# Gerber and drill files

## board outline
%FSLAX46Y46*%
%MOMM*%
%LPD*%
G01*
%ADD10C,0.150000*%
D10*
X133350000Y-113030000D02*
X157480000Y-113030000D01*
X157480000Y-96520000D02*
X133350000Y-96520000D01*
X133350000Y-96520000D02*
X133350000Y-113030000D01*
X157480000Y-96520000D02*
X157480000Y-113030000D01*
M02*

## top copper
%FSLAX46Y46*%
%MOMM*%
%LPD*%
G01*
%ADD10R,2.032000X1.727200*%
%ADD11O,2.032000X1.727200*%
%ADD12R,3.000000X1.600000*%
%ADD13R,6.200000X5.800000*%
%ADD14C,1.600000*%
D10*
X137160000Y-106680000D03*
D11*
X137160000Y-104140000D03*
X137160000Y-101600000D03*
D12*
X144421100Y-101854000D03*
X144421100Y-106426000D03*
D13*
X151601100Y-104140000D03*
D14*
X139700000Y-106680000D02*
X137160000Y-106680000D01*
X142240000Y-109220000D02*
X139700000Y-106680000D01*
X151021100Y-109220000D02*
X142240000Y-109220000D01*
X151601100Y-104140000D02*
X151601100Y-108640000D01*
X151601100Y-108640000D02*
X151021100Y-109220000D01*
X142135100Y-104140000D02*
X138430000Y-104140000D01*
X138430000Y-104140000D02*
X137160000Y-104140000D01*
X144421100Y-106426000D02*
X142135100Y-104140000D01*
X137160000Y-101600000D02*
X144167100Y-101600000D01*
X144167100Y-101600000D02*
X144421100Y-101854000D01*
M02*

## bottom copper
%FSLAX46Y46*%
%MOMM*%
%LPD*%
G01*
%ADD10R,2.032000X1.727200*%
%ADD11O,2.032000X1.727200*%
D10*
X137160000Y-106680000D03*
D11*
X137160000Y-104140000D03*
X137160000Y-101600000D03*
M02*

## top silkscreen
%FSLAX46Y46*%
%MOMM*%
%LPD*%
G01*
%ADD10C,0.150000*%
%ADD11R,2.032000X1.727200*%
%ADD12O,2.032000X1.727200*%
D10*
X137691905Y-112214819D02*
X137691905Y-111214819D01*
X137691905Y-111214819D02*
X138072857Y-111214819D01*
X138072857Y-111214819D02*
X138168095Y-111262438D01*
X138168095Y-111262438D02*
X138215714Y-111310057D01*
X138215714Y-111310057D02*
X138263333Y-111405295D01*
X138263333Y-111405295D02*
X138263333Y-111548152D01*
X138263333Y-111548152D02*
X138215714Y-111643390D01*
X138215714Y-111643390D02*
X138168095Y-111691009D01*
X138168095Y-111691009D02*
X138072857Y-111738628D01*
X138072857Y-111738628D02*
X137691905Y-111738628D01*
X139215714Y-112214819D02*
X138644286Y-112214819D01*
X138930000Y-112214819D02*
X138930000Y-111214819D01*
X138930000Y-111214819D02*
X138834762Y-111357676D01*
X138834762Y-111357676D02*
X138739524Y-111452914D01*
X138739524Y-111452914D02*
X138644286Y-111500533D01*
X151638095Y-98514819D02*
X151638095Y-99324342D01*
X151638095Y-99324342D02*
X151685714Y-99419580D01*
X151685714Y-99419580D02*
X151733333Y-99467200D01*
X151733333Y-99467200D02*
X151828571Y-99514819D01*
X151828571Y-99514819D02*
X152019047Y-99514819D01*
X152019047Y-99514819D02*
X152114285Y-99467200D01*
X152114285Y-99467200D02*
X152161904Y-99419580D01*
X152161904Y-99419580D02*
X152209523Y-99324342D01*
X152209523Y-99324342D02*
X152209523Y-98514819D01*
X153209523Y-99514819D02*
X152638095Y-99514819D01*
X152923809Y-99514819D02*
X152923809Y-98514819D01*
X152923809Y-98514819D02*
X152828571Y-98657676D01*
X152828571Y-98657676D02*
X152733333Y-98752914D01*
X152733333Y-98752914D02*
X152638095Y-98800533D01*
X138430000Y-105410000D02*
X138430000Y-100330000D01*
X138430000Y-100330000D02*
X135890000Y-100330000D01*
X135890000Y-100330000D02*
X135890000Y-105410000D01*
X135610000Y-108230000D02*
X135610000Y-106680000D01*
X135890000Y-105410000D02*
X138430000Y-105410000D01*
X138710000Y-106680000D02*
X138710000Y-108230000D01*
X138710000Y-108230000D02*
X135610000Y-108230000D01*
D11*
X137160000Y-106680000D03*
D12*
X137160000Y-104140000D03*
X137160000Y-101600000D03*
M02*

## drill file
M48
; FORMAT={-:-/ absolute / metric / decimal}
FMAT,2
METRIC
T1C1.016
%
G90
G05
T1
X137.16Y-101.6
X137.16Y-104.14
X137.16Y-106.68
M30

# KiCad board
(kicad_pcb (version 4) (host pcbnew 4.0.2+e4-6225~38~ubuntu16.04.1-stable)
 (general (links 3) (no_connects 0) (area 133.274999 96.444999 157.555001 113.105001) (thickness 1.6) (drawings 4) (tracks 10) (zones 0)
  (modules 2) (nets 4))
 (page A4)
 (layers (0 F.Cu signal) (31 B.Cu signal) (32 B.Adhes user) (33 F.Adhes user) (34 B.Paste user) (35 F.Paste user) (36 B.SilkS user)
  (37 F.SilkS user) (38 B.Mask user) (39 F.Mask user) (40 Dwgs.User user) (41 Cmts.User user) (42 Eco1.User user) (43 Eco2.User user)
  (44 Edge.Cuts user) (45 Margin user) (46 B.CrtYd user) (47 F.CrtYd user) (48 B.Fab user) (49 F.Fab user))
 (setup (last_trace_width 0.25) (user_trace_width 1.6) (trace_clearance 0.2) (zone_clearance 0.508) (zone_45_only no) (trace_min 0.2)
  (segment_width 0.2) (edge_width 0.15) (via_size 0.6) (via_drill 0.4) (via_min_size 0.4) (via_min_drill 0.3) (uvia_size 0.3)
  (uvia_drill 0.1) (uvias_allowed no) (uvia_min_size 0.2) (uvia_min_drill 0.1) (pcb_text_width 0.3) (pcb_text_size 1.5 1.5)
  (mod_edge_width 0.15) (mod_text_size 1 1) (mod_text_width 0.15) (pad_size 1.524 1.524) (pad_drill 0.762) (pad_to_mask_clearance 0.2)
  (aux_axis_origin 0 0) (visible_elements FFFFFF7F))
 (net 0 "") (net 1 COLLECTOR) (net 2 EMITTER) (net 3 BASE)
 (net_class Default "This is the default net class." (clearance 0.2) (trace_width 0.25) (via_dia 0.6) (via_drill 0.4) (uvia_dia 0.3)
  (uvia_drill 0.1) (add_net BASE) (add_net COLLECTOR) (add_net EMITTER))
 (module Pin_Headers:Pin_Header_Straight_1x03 (layer F.Cu) (at 137.16 106.68 180)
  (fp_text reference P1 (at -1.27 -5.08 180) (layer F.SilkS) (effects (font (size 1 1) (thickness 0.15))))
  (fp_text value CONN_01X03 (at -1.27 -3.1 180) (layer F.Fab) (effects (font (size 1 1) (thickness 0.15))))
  (fp_line (start -1.27 1.27) (end -1.27 6.35) (layer F.SilkS) (width 0.15))
  (fp_line (start -1.27 6.35) (end 1.27 6.35) (layer F.SilkS) (width 0.15))
  (fp_line (start 1.27 6.35) (end 1.27 1.27) (layer F.SilkS) (width 0.15))
  (fp_line (start 1.55 -1.55) (end 1.55 0) (layer F.SilkS) (width 0.15))
  (fp_line (start 1.27 1.27) (end -1.27 1.27) (layer F.SilkS) (width 0.15))
  (fp_line (start -1.55 0) (end -1.55 -1.55) (layer F.SilkS) (width 0.15))
  (fp_line (start -1.55 -1.55) (end 1.55 -1.55) (layer F.SilkS) (width 0.15))
  (pad 1 thru_hole rect (at 0 0 180) (size 2.032 1.7272) (drill 1.016) (layers *.Cu *.Mask F.SilkS) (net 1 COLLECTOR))
  (pad 2 thru_hole oval (at 0 2.54 180) (size 2.032 1.7272) (drill 1.016) (layers *.Cu *.Mask F.SilkS) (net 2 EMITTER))
  (pad 3 thru_hole oval (at 0 5.08 180) (size 2.032 1.7272) (drill 1.016) (layers *.Cu *.Mask F.SilkS) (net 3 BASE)))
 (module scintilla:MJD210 (layer F.Cu) (at 148.5011 104.14 180)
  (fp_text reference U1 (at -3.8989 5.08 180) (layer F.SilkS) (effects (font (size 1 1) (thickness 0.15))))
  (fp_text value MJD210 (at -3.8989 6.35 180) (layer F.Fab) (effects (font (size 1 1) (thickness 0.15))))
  (pad 1 smd rect (at 4.08 2.286 180) (size 3 1.6) (layers F.Cu F.Paste F.Mask) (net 3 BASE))
  (pad 3 smd rect (at 4.08 -2.286 180) (size 3 1.6) (layers F.Cu F.Paste F.Mask) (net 2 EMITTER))
  (pad 4 smd rect (at -3.1 0 180) (size 6.2 5.8) (layers F.Cu F.Paste F.Mask) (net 1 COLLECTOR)))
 (gr_line (start 133.35 113.03) (end 157.48 113.03) (layer Edge.Cuts) (width 0.15))
 (gr_line (start 157.48 96.52) (end 133.35 96.52) (layer Edge.Cuts) (width 0.15))
 (gr_line (start 133.35 96.52) (end 133.35 113.03) (layer Edge.Cuts) (width 0.15))
 (gr_line (start 157.48 96.52) (end 157.48 113.03) (layer Edge.Cuts) (width 0.15))
 (segment (start 139.7 106.68) (end 137.16 106.68) (width 1.6) (layer F.Cu) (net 1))
 (segment (start 142.24 109.22) (end 139.7 106.68) (width 1.6) (layer F.Cu) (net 1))
 (segment (start 151.0211 109.22) (end 142.24 109.22) (width 1.6) (layer F.Cu) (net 1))
 (segment (start 151.6011 104.14) (end 151.6011 108.64) (width 1.6) (layer F.Cu) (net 1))
 (segment (start 151.6011 108.64) (end 151.0211 109.22) (width 1.6) (layer F.Cu) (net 1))
 (segment (start 142.1351 104.14) (end 138.43 104.14) (width 1.6) (layer F.Cu) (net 2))
 (segment (start 138.43 104.14) (end 137.16 104.14) (width 1.6) (layer F.Cu) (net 2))
 (segment (start 144.4211 106.426) (end 142.1351 104.14) (width 1.6) (layer F.Cu) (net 2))
 (segment (start 137.16 101.6) (end 144.1671 101.6) (width 1.6) (layer F.Cu) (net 3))
 (segment (start 144.1671 101.6) (end 144.4211 101.854) (width 1.6) (layer F.Cu) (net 3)))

